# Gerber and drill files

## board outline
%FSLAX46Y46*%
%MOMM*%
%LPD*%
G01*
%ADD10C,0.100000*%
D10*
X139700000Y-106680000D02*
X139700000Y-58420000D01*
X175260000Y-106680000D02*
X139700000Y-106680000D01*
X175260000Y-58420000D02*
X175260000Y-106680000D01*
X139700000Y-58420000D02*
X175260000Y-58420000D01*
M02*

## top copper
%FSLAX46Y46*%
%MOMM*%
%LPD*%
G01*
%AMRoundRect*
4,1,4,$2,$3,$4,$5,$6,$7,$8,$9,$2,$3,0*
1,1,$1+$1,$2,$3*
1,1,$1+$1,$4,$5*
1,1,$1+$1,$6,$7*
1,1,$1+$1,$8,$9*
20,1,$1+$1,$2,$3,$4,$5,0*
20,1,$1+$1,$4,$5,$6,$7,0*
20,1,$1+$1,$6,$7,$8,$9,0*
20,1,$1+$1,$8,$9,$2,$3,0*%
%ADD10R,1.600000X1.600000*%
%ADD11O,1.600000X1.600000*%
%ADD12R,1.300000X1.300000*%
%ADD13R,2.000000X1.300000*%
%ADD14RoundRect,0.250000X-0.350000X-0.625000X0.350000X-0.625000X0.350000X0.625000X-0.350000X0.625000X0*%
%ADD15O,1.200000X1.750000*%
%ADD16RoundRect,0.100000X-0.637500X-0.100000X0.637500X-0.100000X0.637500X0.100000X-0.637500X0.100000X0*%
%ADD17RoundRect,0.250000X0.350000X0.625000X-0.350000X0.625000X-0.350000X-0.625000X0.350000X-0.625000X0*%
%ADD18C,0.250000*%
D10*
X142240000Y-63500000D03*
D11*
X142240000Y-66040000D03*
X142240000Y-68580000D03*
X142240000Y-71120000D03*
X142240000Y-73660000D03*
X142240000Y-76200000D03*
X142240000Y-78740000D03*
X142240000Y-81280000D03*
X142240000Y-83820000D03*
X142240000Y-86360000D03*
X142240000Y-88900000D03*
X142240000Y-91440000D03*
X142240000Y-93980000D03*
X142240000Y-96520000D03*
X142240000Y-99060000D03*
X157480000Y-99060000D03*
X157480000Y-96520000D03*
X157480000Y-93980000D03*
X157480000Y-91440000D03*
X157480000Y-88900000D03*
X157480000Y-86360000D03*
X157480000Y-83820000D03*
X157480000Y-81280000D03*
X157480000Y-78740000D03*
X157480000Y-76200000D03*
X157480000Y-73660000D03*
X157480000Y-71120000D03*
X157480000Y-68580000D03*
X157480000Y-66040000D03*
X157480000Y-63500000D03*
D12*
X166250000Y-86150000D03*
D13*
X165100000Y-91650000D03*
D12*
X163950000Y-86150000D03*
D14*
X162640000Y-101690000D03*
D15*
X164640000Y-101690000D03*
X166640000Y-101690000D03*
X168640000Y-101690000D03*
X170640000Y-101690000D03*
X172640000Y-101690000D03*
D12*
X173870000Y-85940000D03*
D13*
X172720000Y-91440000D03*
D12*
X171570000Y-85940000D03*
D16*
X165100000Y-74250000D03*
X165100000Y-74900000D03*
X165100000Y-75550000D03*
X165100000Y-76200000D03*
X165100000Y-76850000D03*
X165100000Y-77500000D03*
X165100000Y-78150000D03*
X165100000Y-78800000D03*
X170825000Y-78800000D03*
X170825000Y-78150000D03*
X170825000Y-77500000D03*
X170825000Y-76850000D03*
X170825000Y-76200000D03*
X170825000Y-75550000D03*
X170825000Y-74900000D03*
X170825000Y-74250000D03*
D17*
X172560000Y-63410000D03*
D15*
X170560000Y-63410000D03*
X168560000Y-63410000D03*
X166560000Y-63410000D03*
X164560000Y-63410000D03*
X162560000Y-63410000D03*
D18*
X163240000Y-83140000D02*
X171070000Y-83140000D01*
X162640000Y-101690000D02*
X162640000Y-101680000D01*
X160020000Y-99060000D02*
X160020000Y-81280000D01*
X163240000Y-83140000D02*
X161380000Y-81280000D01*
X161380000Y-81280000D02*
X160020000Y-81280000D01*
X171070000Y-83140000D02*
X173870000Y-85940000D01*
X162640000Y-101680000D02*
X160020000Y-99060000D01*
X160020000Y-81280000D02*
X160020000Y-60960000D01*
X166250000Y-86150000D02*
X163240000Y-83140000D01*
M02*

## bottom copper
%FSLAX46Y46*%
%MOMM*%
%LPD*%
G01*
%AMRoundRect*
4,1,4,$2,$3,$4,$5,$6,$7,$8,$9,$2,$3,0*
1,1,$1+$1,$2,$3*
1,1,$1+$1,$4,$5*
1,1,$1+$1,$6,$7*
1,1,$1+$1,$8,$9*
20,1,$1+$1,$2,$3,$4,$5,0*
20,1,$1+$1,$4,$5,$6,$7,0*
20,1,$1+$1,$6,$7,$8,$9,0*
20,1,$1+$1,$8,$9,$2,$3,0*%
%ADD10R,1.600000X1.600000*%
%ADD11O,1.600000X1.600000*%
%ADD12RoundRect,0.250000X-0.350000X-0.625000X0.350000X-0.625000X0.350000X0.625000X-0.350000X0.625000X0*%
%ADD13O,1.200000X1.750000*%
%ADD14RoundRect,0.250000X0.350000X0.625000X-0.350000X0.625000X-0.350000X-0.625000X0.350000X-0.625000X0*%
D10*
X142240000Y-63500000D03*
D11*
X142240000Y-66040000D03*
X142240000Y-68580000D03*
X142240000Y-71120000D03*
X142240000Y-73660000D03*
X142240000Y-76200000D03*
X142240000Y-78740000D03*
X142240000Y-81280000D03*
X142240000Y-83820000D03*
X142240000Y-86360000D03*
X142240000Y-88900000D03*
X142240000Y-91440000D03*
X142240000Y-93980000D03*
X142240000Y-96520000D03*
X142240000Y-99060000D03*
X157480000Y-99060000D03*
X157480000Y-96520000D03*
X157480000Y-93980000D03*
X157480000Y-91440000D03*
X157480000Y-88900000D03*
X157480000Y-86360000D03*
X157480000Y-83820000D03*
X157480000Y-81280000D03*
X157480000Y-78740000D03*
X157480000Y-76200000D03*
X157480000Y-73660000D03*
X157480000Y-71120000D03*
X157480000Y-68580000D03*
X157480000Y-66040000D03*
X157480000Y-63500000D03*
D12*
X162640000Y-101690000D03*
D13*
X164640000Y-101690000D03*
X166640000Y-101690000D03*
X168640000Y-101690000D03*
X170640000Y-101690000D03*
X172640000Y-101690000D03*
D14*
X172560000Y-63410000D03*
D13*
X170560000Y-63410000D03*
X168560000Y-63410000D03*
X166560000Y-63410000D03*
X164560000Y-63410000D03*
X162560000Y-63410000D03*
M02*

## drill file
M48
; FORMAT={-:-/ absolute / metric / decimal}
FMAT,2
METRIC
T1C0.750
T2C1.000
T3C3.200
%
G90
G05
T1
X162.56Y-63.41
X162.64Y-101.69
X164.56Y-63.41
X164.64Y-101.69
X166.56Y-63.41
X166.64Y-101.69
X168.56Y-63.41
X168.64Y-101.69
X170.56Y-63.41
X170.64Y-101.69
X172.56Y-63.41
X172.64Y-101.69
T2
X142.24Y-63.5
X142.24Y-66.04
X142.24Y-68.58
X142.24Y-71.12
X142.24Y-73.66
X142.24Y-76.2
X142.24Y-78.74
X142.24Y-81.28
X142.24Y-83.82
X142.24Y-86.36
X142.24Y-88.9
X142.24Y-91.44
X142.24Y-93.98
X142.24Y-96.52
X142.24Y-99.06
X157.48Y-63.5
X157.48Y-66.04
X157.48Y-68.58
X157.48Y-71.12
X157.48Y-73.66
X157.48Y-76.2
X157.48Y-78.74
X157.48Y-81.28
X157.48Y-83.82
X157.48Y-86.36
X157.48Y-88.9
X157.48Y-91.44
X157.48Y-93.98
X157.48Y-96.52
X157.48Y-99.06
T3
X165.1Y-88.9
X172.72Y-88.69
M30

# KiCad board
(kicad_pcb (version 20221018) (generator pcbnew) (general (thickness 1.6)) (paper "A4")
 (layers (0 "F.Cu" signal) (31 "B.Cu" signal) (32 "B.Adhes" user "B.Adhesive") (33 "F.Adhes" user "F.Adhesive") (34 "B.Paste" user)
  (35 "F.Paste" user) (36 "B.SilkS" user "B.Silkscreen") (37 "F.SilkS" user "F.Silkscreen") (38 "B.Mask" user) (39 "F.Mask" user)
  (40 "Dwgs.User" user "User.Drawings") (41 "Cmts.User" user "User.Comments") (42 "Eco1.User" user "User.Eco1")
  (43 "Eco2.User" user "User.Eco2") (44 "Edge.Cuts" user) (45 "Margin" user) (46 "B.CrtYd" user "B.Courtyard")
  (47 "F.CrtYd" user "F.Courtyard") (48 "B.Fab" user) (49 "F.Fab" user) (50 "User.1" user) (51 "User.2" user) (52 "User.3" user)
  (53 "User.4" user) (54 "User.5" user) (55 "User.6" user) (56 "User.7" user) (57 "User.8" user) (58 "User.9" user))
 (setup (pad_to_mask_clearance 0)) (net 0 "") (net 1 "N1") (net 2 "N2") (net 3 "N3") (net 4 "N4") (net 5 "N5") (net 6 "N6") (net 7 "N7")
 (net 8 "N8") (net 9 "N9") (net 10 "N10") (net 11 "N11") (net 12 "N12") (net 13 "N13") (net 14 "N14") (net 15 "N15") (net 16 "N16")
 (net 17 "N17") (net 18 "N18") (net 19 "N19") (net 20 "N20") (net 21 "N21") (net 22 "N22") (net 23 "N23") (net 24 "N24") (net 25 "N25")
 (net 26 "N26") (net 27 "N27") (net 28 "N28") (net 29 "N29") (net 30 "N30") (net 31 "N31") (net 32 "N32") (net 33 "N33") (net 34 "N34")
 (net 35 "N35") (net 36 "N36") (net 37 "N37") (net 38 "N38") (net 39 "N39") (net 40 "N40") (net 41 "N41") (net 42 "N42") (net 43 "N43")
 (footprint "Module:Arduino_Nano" (layer "F.Cu") (at 142.24 63.5)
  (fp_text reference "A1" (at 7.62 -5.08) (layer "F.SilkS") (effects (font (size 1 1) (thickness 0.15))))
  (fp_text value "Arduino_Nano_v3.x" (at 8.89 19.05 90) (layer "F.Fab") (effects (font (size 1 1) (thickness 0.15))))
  (pad "1" thru_hole rect (at 0 0) (size 1.6 1.6) (drill 1) (layers "*.Cu" "*.Mask") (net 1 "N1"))
  (pad "2" thru_hole oval (at 0 2.54) (size 1.6 1.6) (drill 1) (layers "*.Cu" "*.Mask") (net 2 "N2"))
  (pad "3" thru_hole oval (at 0 5.08) (size 1.6 1.6) (drill 1) (layers "*.Cu" "*.Mask") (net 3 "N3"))
  (pad "4" thru_hole oval (at 0 7.62) (size 1.6 1.6) (drill 1) (layers "*.Cu" "*.Mask") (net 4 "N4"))
  (pad "5" thru_hole oval (at 0 10.16) (size 1.6 1.6) (drill 1) (layers "*.Cu" "*.Mask") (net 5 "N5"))
  (pad "6" thru_hole oval (at 0 12.7) (size 1.6 1.6) (drill 1) (layers "*.Cu" "*.Mask") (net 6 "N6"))
  (pad "7" thru_hole oval (at 0 15.24) (size 1.6 1.6) (drill 1) (layers "*.Cu" "*.Mask") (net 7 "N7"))
  (pad "8" thru_hole oval (at 0 17.78) (size 1.6 1.6) (drill 1) (layers "*.Cu" "*.Mask") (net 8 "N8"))
  (pad "9" thru_hole oval (at 0 20.32) (size 1.6 1.6) (drill 1) (layers "*.Cu" "*.Mask") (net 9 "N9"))
  (pad "10" thru_hole oval (at 0 22.86) (size 1.6 1.6) (drill 1) (layers "*.Cu" "*.Mask") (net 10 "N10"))
  (pad "11" thru_hole oval (at 0 25.4) (size 1.6 1.6) (drill 1) (layers "*.Cu" "*.Mask") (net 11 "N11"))
  (pad "12" thru_hole oval (at 0 27.94) (size 1.6 1.6) (drill 1) (layers "*.Cu" "*.Mask") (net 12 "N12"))
  (pad "13" thru_hole oval (at 0 30.48) (size 1.6 1.6) (drill 1) (layers "*.Cu" "*.Mask") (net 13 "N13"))
  (pad "14" thru_hole oval (at 0 33.02) (size 1.6 1.6) (drill 1) (layers "*.Cu" "*.Mask") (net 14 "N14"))
  (pad "15" thru_hole oval (at 0 35.56) (size 1.6 1.6) (drill 1) (layers "*.Cu" "*.Mask") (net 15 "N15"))
  (pad "16" thru_hole oval (at 15.24 35.56) (size 1.6 1.6) (drill 1) (layers "*.Cu" "*.Mask") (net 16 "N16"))
  (pad "17" thru_hole oval (at 15.24 33.02) (size 1.6 1.6) (drill 1) (layers "*.Cu" "*.Mask") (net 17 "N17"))
  (pad "18" thru_hole oval (at 15.24 30.48) (size 1.6 1.6) (drill 1) (layers "*.Cu" "*.Mask") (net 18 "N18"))
  (pad "19" thru_hole oval (at 15.24 27.94) (size 1.6 1.6) (drill 1) (layers "*.Cu" "*.Mask") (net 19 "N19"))
  (pad "20" thru_hole oval (at 15.24 25.4) (size 1.6 1.6) (drill 1) (layers "*.Cu" "*.Mask") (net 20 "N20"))
  (pad "21" thru_hole oval (at 15.24 22.86) (size 1.6 1.6) (drill 1) (layers "*.Cu" "*.Mask") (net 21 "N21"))
  (pad "22" thru_hole oval (at 15.24 20.32) (size 1.6 1.6) (drill 1) (layers "*.Cu" "*.Mask") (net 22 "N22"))
  (pad "23" thru_hole oval (at 15.24 17.78) (size 1.6 1.6) (drill 1) (layers "*.Cu" "*.Mask") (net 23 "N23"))
  (pad "24" thru_hole oval (at 15.24 15.24) (size 1.6 1.6) (drill 1) (layers "*.Cu" "*.Mask") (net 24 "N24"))
  (pad "25" thru_hole oval (at 15.24 12.7) (size 1.6 1.6) (drill 1) (layers "*.Cu" "*.Mask") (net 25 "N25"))
  (pad "26" thru_hole oval (at 15.24 10.16) (size 1.6 1.6) (drill 1) (layers "*.Cu" "*.Mask") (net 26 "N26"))
  (pad "27" thru_hole oval (at 15.24 7.62) (size 1.6 1.6) (drill 1) (layers "*.Cu" "*.Mask") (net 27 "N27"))
  (pad "28" thru_hole oval (at 15.24 5.08) (size 1.6 1.6) (drill 1) (layers "*.Cu" "*.Mask") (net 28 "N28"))
  (pad "29" thru_hole oval (at 15.24 2.54) (size 1.6 1.6) (drill 1) (layers "*.Cu" "*.Mask") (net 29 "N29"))
  (pad "30" thru_hole oval (at 15.24 0) (size 1.6 1.6) (drill 1) (layers "*.Cu" "*.Mask") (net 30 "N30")))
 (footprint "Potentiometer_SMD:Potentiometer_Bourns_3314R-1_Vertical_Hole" (layer "F.Cu") (at 165.1 88.9)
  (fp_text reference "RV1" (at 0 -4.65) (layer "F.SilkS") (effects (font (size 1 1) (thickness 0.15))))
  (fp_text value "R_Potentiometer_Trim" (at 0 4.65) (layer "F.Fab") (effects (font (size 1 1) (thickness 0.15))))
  (pad "" np_thru_hole circle (at 0 0) (size 3.2 3.2) (drill 3.2) (layers "*.Cu" "*.Mask"))
  (pad "1" smd rect (at 1.15 -2.75) (size 1.3 1.3) (layers "F.Cu" "F.Paste" "F.Mask") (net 30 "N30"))
  (pad "2" smd rect (at 0 2.75) (size 2 1.3) (layers "F.Cu" "F.Paste" "F.Mask") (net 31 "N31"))
  (pad "3" smd rect (at -1.15 -2.75) (size 1.3 1.3) (layers "F.Cu" "F.Paste" "F.Mask") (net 29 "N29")))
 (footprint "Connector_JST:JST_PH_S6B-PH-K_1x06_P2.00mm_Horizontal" (layer "F.Cu") (at 162.64 101.69)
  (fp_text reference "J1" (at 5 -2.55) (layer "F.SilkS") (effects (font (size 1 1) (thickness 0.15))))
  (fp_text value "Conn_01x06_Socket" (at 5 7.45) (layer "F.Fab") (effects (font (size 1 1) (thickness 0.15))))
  (pad "1" thru_hole roundrect (at 0 0) (size 1.2 1.75) (drill 0.75) (layers "*.Cu" "*.Mask") (roundrect_rratio 0.208333) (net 30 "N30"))
  (pad "2" thru_hole oval (at 2 0) (size 1.2 1.75) (drill 0.75) (layers "*.Cu" "*.Mask") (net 29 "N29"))
  (pad "3" thru_hole oval (at 4 0) (size 1.2 1.75) (drill 0.75) (layers "*.Cu" "*.Mask") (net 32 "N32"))
  (pad "4" thru_hole oval (at 6 0) (size 1.2 1.75) (drill 0.75) (layers "*.Cu" "*.Mask") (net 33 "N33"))
  (pad "5" thru_hole oval (at 8 0) (size 1.2 1.75) (drill 0.75) (layers "*.Cu" "*.Mask") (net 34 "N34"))
  (pad "6" thru_hole oval (at 10 0) (size 1.2 1.75) (drill 0.75) (layers "*.Cu" "*.Mask") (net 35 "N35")))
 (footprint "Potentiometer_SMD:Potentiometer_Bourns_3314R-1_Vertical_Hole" (layer "F.Cu") (at 172.72 88.69)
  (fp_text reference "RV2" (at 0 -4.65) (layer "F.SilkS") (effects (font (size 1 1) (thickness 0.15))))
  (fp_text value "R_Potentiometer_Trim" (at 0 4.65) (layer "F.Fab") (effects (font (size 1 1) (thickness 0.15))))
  (pad "" np_thru_hole circle (at 0 0) (size 3.2 3.2) (drill 3.2) (layers "*.Cu" "*.Mask"))
  (pad "1" smd rect (at 1.15 -2.75) (size 1.3 1.3) (layers "F.Cu" "F.Paste" "F.Mask") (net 30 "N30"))
  (pad "2" smd rect (at 0 2.75) (size 2 1.3) (layers "F.Cu" "F.Paste" "F.Mask") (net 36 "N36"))
  (pad "3" smd rect (at -1.15 -2.75) (size 1.3 1.3) (layers "F.Cu" "F.Paste" "F.Mask") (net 29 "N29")))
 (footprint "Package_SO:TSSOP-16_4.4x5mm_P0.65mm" (layer "F.Cu") (at 167.9625 76.525)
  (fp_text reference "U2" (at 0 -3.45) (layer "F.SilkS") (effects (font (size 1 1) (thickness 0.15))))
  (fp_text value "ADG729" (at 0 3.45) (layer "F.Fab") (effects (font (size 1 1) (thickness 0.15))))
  (pad "1" smd roundrect (at -2.8625 -2.275) (size 1.475 0.4) (layers "F.Cu" "F.Paste" "F.Mask") (roundrect_rratio 0.25) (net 23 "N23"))
  (pad "2" smd roundrect (at -2.8625 -1.625) (size 1.475 0.4) (layers "F.Cu" "F.Paste" "F.Mask") (roundrect_rratio 0.25) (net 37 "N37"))
  (pad "3" smd roundrect (at -2.8625 -0.975) (size 1.475 0.4) (layers "F.Cu" "F.Paste" "F.Mask") (roundrect_rratio 0.25) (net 24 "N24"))
  (pad "4" smd roundrect (at -2.8625 -0.325) (size 1.475 0.4) (layers "F.Cu" "F.Paste" "F.Mask") (roundrect_rratio 0.25) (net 32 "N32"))
  (pad "5" smd roundrect (at -2.8625 0.325) (size 1.475 0.4) (layers "F.Cu" "F.Paste" "F.Mask") (roundrect_rratio 0.25) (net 36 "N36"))
  (pad "6" smd roundrect (at -2.8625 0.975) (size 1.475 0.4) (layers "F.Cu" "F.Paste" "F.Mask") (roundrect_rratio 0.25) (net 31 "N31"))
  (pad "7" smd roundrect (at -2.8625 1.625) (size 1.475 0.4) (layers "F.Cu" "F.Paste" "F.Mask") (roundrect_rratio 0.25) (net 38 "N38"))
  (pad "8" smd roundrect (at -2.8625 2.275) (size 1.475 0.4) (layers "F.Cu" "F.Paste" "F.Mask") (roundrect_rratio 0.25) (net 34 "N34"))
  (pad "9" smd roundrect (at 2.8625 2.275) (size 1.475 0.4) (layers "F.Cu" "F.Paste" "F.Mask") (roundrect_rratio 0.25) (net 35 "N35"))
  (pad "10" smd roundrect (at 2.8625 1.625) (size 1.475 0.4) (layers "F.Cu" "F.Paste" "F.Mask") (roundrect_rratio 0.25) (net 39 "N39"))
  (pad "11" smd roundrect (at 2.8625 0.975) (size 1.475 0.4) (layers "F.Cu" "F.Paste" "F.Mask") (roundrect_rratio 0.25) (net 31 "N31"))
  (pad "12" smd roundrect (at 2.8625 0.325) (size 1.475 0.4) (layers "F.Cu" "F.Paste" "F.Mask") (roundrect_rratio 0.25) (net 36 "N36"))
  (pad "13" smd roundrect (at 2.8625 -0.325) (size 1.475 0.4) (layers "F.Cu" "F.Paste" "F.Mask") (roundrect_rratio 0.25) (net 33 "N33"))
  (pad "14" smd roundrect (at 2.8625 -0.975) (size 1.475 0.4) (layers "F.Cu" "F.Paste" "F.Mask") (roundrect_rratio 0.25) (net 30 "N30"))
  (pad "15" smd roundrect (at 2.8625 -1.625) (size 1.475 0.4) (layers "F.Cu" "F.Paste" "F.Mask") (roundrect_rratio 0.25) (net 29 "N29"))
  (pad "16" smd roundrect (at 2.8625 -2.275) (size 1.475 0.4) (layers "F.Cu" "F.Paste" "F.Mask") (roundrect_rratio 0.25) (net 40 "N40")))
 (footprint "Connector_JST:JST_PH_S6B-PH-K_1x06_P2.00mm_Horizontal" (layer "F.Cu") (at 172.56 63.41 180)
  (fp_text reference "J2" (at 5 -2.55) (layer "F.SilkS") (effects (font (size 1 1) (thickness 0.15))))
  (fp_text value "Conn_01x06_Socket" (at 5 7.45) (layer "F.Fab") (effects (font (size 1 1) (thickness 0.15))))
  (pad "1" thru_hole roundrect (at 0 0 180) (size 1.2 1.75) (drill 0.75) (layers "*.Cu" "*.Mask") (roundrect_rratio 0.208333) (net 8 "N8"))
  (pad "2" thru_hole oval (at 2 0 180) (size 1.2 1.75) (drill 0.75) (layers "*.Cu" "*.Mask") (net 10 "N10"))
  (pad "3" thru_hole oval (at 4 0 180) (size 1.2 1.75) (drill 0.75) (layers "*.Cu" "*.Mask") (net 9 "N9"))
  (pad "4" thru_hole oval (at 6 0 180) (size 1.2 1.75) (drill 0.75) (layers "*.Cu" "*.Mask") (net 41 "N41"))
  (pad "5" thru_hole oval (at 8 0 180) (size 1.2 1.75) (drill 0.75) (layers "*.Cu" "*.Mask") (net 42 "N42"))
  (pad "6" thru_hole oval (at 10 0 180) (size 1.2 1.75) (drill 0.75) (layers "*.Cu" "*.Mask") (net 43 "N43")))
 (gr_line (start 139.7 106.68) (end 139.7 58.42) (stroke (width 0.1) (type default)) (layer "Edge.Cuts"))
 (gr_line (start 175.26 106.68) (end 139.7 106.68) (stroke (width 0.1) (type default)) (layer "Edge.Cuts"))
 (gr_line (start 175.26 58.42) (end 175.26 106.68) (stroke (width 0.1) (type default)) (layer "Edge.Cuts"))
 (gr_line (start 139.7 58.42) (end 175.26 58.42) (stroke (width 0.1) (type default)) (layer "Edge.Cuts"))
 (segment (start 163.24 83.14) (end 171.07 83.14) (width 0.25) (layer "F.Cu") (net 30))
 (segment (start 162.64 101.69) (end 162.64 101.68) (width 0.25) (layer "F.Cu") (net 30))
 (segment (start 160.02 99.06) (end 160.02 81.28) (width 0.25) (layer "F.Cu") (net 30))
 (segment (start 163.24 83.14) (end 161.38 81.28) (width 0.25) (layer "F.Cu") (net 30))
 (segment (start 161.38 81.28) (end 160.02 81.28) (width 0.25) (layer "F.Cu") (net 30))
 (segment (start 171.07 83.14) (end 173.87 85.94) (width 0.25) (layer "F.Cu") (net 30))
 (segment (start 162.64 101.68) (end 160.02 99.06) (width 0.25) (layer "F.Cu") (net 30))
 (segment (start 160.02 81.28) (end 160.02 60.96) (width 0.25) (layer "F.Cu") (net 30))
 (segment (start 166.25 86.15) (end 163.24 83.14) (width 0.25) (layer "F.Cu") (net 30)))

